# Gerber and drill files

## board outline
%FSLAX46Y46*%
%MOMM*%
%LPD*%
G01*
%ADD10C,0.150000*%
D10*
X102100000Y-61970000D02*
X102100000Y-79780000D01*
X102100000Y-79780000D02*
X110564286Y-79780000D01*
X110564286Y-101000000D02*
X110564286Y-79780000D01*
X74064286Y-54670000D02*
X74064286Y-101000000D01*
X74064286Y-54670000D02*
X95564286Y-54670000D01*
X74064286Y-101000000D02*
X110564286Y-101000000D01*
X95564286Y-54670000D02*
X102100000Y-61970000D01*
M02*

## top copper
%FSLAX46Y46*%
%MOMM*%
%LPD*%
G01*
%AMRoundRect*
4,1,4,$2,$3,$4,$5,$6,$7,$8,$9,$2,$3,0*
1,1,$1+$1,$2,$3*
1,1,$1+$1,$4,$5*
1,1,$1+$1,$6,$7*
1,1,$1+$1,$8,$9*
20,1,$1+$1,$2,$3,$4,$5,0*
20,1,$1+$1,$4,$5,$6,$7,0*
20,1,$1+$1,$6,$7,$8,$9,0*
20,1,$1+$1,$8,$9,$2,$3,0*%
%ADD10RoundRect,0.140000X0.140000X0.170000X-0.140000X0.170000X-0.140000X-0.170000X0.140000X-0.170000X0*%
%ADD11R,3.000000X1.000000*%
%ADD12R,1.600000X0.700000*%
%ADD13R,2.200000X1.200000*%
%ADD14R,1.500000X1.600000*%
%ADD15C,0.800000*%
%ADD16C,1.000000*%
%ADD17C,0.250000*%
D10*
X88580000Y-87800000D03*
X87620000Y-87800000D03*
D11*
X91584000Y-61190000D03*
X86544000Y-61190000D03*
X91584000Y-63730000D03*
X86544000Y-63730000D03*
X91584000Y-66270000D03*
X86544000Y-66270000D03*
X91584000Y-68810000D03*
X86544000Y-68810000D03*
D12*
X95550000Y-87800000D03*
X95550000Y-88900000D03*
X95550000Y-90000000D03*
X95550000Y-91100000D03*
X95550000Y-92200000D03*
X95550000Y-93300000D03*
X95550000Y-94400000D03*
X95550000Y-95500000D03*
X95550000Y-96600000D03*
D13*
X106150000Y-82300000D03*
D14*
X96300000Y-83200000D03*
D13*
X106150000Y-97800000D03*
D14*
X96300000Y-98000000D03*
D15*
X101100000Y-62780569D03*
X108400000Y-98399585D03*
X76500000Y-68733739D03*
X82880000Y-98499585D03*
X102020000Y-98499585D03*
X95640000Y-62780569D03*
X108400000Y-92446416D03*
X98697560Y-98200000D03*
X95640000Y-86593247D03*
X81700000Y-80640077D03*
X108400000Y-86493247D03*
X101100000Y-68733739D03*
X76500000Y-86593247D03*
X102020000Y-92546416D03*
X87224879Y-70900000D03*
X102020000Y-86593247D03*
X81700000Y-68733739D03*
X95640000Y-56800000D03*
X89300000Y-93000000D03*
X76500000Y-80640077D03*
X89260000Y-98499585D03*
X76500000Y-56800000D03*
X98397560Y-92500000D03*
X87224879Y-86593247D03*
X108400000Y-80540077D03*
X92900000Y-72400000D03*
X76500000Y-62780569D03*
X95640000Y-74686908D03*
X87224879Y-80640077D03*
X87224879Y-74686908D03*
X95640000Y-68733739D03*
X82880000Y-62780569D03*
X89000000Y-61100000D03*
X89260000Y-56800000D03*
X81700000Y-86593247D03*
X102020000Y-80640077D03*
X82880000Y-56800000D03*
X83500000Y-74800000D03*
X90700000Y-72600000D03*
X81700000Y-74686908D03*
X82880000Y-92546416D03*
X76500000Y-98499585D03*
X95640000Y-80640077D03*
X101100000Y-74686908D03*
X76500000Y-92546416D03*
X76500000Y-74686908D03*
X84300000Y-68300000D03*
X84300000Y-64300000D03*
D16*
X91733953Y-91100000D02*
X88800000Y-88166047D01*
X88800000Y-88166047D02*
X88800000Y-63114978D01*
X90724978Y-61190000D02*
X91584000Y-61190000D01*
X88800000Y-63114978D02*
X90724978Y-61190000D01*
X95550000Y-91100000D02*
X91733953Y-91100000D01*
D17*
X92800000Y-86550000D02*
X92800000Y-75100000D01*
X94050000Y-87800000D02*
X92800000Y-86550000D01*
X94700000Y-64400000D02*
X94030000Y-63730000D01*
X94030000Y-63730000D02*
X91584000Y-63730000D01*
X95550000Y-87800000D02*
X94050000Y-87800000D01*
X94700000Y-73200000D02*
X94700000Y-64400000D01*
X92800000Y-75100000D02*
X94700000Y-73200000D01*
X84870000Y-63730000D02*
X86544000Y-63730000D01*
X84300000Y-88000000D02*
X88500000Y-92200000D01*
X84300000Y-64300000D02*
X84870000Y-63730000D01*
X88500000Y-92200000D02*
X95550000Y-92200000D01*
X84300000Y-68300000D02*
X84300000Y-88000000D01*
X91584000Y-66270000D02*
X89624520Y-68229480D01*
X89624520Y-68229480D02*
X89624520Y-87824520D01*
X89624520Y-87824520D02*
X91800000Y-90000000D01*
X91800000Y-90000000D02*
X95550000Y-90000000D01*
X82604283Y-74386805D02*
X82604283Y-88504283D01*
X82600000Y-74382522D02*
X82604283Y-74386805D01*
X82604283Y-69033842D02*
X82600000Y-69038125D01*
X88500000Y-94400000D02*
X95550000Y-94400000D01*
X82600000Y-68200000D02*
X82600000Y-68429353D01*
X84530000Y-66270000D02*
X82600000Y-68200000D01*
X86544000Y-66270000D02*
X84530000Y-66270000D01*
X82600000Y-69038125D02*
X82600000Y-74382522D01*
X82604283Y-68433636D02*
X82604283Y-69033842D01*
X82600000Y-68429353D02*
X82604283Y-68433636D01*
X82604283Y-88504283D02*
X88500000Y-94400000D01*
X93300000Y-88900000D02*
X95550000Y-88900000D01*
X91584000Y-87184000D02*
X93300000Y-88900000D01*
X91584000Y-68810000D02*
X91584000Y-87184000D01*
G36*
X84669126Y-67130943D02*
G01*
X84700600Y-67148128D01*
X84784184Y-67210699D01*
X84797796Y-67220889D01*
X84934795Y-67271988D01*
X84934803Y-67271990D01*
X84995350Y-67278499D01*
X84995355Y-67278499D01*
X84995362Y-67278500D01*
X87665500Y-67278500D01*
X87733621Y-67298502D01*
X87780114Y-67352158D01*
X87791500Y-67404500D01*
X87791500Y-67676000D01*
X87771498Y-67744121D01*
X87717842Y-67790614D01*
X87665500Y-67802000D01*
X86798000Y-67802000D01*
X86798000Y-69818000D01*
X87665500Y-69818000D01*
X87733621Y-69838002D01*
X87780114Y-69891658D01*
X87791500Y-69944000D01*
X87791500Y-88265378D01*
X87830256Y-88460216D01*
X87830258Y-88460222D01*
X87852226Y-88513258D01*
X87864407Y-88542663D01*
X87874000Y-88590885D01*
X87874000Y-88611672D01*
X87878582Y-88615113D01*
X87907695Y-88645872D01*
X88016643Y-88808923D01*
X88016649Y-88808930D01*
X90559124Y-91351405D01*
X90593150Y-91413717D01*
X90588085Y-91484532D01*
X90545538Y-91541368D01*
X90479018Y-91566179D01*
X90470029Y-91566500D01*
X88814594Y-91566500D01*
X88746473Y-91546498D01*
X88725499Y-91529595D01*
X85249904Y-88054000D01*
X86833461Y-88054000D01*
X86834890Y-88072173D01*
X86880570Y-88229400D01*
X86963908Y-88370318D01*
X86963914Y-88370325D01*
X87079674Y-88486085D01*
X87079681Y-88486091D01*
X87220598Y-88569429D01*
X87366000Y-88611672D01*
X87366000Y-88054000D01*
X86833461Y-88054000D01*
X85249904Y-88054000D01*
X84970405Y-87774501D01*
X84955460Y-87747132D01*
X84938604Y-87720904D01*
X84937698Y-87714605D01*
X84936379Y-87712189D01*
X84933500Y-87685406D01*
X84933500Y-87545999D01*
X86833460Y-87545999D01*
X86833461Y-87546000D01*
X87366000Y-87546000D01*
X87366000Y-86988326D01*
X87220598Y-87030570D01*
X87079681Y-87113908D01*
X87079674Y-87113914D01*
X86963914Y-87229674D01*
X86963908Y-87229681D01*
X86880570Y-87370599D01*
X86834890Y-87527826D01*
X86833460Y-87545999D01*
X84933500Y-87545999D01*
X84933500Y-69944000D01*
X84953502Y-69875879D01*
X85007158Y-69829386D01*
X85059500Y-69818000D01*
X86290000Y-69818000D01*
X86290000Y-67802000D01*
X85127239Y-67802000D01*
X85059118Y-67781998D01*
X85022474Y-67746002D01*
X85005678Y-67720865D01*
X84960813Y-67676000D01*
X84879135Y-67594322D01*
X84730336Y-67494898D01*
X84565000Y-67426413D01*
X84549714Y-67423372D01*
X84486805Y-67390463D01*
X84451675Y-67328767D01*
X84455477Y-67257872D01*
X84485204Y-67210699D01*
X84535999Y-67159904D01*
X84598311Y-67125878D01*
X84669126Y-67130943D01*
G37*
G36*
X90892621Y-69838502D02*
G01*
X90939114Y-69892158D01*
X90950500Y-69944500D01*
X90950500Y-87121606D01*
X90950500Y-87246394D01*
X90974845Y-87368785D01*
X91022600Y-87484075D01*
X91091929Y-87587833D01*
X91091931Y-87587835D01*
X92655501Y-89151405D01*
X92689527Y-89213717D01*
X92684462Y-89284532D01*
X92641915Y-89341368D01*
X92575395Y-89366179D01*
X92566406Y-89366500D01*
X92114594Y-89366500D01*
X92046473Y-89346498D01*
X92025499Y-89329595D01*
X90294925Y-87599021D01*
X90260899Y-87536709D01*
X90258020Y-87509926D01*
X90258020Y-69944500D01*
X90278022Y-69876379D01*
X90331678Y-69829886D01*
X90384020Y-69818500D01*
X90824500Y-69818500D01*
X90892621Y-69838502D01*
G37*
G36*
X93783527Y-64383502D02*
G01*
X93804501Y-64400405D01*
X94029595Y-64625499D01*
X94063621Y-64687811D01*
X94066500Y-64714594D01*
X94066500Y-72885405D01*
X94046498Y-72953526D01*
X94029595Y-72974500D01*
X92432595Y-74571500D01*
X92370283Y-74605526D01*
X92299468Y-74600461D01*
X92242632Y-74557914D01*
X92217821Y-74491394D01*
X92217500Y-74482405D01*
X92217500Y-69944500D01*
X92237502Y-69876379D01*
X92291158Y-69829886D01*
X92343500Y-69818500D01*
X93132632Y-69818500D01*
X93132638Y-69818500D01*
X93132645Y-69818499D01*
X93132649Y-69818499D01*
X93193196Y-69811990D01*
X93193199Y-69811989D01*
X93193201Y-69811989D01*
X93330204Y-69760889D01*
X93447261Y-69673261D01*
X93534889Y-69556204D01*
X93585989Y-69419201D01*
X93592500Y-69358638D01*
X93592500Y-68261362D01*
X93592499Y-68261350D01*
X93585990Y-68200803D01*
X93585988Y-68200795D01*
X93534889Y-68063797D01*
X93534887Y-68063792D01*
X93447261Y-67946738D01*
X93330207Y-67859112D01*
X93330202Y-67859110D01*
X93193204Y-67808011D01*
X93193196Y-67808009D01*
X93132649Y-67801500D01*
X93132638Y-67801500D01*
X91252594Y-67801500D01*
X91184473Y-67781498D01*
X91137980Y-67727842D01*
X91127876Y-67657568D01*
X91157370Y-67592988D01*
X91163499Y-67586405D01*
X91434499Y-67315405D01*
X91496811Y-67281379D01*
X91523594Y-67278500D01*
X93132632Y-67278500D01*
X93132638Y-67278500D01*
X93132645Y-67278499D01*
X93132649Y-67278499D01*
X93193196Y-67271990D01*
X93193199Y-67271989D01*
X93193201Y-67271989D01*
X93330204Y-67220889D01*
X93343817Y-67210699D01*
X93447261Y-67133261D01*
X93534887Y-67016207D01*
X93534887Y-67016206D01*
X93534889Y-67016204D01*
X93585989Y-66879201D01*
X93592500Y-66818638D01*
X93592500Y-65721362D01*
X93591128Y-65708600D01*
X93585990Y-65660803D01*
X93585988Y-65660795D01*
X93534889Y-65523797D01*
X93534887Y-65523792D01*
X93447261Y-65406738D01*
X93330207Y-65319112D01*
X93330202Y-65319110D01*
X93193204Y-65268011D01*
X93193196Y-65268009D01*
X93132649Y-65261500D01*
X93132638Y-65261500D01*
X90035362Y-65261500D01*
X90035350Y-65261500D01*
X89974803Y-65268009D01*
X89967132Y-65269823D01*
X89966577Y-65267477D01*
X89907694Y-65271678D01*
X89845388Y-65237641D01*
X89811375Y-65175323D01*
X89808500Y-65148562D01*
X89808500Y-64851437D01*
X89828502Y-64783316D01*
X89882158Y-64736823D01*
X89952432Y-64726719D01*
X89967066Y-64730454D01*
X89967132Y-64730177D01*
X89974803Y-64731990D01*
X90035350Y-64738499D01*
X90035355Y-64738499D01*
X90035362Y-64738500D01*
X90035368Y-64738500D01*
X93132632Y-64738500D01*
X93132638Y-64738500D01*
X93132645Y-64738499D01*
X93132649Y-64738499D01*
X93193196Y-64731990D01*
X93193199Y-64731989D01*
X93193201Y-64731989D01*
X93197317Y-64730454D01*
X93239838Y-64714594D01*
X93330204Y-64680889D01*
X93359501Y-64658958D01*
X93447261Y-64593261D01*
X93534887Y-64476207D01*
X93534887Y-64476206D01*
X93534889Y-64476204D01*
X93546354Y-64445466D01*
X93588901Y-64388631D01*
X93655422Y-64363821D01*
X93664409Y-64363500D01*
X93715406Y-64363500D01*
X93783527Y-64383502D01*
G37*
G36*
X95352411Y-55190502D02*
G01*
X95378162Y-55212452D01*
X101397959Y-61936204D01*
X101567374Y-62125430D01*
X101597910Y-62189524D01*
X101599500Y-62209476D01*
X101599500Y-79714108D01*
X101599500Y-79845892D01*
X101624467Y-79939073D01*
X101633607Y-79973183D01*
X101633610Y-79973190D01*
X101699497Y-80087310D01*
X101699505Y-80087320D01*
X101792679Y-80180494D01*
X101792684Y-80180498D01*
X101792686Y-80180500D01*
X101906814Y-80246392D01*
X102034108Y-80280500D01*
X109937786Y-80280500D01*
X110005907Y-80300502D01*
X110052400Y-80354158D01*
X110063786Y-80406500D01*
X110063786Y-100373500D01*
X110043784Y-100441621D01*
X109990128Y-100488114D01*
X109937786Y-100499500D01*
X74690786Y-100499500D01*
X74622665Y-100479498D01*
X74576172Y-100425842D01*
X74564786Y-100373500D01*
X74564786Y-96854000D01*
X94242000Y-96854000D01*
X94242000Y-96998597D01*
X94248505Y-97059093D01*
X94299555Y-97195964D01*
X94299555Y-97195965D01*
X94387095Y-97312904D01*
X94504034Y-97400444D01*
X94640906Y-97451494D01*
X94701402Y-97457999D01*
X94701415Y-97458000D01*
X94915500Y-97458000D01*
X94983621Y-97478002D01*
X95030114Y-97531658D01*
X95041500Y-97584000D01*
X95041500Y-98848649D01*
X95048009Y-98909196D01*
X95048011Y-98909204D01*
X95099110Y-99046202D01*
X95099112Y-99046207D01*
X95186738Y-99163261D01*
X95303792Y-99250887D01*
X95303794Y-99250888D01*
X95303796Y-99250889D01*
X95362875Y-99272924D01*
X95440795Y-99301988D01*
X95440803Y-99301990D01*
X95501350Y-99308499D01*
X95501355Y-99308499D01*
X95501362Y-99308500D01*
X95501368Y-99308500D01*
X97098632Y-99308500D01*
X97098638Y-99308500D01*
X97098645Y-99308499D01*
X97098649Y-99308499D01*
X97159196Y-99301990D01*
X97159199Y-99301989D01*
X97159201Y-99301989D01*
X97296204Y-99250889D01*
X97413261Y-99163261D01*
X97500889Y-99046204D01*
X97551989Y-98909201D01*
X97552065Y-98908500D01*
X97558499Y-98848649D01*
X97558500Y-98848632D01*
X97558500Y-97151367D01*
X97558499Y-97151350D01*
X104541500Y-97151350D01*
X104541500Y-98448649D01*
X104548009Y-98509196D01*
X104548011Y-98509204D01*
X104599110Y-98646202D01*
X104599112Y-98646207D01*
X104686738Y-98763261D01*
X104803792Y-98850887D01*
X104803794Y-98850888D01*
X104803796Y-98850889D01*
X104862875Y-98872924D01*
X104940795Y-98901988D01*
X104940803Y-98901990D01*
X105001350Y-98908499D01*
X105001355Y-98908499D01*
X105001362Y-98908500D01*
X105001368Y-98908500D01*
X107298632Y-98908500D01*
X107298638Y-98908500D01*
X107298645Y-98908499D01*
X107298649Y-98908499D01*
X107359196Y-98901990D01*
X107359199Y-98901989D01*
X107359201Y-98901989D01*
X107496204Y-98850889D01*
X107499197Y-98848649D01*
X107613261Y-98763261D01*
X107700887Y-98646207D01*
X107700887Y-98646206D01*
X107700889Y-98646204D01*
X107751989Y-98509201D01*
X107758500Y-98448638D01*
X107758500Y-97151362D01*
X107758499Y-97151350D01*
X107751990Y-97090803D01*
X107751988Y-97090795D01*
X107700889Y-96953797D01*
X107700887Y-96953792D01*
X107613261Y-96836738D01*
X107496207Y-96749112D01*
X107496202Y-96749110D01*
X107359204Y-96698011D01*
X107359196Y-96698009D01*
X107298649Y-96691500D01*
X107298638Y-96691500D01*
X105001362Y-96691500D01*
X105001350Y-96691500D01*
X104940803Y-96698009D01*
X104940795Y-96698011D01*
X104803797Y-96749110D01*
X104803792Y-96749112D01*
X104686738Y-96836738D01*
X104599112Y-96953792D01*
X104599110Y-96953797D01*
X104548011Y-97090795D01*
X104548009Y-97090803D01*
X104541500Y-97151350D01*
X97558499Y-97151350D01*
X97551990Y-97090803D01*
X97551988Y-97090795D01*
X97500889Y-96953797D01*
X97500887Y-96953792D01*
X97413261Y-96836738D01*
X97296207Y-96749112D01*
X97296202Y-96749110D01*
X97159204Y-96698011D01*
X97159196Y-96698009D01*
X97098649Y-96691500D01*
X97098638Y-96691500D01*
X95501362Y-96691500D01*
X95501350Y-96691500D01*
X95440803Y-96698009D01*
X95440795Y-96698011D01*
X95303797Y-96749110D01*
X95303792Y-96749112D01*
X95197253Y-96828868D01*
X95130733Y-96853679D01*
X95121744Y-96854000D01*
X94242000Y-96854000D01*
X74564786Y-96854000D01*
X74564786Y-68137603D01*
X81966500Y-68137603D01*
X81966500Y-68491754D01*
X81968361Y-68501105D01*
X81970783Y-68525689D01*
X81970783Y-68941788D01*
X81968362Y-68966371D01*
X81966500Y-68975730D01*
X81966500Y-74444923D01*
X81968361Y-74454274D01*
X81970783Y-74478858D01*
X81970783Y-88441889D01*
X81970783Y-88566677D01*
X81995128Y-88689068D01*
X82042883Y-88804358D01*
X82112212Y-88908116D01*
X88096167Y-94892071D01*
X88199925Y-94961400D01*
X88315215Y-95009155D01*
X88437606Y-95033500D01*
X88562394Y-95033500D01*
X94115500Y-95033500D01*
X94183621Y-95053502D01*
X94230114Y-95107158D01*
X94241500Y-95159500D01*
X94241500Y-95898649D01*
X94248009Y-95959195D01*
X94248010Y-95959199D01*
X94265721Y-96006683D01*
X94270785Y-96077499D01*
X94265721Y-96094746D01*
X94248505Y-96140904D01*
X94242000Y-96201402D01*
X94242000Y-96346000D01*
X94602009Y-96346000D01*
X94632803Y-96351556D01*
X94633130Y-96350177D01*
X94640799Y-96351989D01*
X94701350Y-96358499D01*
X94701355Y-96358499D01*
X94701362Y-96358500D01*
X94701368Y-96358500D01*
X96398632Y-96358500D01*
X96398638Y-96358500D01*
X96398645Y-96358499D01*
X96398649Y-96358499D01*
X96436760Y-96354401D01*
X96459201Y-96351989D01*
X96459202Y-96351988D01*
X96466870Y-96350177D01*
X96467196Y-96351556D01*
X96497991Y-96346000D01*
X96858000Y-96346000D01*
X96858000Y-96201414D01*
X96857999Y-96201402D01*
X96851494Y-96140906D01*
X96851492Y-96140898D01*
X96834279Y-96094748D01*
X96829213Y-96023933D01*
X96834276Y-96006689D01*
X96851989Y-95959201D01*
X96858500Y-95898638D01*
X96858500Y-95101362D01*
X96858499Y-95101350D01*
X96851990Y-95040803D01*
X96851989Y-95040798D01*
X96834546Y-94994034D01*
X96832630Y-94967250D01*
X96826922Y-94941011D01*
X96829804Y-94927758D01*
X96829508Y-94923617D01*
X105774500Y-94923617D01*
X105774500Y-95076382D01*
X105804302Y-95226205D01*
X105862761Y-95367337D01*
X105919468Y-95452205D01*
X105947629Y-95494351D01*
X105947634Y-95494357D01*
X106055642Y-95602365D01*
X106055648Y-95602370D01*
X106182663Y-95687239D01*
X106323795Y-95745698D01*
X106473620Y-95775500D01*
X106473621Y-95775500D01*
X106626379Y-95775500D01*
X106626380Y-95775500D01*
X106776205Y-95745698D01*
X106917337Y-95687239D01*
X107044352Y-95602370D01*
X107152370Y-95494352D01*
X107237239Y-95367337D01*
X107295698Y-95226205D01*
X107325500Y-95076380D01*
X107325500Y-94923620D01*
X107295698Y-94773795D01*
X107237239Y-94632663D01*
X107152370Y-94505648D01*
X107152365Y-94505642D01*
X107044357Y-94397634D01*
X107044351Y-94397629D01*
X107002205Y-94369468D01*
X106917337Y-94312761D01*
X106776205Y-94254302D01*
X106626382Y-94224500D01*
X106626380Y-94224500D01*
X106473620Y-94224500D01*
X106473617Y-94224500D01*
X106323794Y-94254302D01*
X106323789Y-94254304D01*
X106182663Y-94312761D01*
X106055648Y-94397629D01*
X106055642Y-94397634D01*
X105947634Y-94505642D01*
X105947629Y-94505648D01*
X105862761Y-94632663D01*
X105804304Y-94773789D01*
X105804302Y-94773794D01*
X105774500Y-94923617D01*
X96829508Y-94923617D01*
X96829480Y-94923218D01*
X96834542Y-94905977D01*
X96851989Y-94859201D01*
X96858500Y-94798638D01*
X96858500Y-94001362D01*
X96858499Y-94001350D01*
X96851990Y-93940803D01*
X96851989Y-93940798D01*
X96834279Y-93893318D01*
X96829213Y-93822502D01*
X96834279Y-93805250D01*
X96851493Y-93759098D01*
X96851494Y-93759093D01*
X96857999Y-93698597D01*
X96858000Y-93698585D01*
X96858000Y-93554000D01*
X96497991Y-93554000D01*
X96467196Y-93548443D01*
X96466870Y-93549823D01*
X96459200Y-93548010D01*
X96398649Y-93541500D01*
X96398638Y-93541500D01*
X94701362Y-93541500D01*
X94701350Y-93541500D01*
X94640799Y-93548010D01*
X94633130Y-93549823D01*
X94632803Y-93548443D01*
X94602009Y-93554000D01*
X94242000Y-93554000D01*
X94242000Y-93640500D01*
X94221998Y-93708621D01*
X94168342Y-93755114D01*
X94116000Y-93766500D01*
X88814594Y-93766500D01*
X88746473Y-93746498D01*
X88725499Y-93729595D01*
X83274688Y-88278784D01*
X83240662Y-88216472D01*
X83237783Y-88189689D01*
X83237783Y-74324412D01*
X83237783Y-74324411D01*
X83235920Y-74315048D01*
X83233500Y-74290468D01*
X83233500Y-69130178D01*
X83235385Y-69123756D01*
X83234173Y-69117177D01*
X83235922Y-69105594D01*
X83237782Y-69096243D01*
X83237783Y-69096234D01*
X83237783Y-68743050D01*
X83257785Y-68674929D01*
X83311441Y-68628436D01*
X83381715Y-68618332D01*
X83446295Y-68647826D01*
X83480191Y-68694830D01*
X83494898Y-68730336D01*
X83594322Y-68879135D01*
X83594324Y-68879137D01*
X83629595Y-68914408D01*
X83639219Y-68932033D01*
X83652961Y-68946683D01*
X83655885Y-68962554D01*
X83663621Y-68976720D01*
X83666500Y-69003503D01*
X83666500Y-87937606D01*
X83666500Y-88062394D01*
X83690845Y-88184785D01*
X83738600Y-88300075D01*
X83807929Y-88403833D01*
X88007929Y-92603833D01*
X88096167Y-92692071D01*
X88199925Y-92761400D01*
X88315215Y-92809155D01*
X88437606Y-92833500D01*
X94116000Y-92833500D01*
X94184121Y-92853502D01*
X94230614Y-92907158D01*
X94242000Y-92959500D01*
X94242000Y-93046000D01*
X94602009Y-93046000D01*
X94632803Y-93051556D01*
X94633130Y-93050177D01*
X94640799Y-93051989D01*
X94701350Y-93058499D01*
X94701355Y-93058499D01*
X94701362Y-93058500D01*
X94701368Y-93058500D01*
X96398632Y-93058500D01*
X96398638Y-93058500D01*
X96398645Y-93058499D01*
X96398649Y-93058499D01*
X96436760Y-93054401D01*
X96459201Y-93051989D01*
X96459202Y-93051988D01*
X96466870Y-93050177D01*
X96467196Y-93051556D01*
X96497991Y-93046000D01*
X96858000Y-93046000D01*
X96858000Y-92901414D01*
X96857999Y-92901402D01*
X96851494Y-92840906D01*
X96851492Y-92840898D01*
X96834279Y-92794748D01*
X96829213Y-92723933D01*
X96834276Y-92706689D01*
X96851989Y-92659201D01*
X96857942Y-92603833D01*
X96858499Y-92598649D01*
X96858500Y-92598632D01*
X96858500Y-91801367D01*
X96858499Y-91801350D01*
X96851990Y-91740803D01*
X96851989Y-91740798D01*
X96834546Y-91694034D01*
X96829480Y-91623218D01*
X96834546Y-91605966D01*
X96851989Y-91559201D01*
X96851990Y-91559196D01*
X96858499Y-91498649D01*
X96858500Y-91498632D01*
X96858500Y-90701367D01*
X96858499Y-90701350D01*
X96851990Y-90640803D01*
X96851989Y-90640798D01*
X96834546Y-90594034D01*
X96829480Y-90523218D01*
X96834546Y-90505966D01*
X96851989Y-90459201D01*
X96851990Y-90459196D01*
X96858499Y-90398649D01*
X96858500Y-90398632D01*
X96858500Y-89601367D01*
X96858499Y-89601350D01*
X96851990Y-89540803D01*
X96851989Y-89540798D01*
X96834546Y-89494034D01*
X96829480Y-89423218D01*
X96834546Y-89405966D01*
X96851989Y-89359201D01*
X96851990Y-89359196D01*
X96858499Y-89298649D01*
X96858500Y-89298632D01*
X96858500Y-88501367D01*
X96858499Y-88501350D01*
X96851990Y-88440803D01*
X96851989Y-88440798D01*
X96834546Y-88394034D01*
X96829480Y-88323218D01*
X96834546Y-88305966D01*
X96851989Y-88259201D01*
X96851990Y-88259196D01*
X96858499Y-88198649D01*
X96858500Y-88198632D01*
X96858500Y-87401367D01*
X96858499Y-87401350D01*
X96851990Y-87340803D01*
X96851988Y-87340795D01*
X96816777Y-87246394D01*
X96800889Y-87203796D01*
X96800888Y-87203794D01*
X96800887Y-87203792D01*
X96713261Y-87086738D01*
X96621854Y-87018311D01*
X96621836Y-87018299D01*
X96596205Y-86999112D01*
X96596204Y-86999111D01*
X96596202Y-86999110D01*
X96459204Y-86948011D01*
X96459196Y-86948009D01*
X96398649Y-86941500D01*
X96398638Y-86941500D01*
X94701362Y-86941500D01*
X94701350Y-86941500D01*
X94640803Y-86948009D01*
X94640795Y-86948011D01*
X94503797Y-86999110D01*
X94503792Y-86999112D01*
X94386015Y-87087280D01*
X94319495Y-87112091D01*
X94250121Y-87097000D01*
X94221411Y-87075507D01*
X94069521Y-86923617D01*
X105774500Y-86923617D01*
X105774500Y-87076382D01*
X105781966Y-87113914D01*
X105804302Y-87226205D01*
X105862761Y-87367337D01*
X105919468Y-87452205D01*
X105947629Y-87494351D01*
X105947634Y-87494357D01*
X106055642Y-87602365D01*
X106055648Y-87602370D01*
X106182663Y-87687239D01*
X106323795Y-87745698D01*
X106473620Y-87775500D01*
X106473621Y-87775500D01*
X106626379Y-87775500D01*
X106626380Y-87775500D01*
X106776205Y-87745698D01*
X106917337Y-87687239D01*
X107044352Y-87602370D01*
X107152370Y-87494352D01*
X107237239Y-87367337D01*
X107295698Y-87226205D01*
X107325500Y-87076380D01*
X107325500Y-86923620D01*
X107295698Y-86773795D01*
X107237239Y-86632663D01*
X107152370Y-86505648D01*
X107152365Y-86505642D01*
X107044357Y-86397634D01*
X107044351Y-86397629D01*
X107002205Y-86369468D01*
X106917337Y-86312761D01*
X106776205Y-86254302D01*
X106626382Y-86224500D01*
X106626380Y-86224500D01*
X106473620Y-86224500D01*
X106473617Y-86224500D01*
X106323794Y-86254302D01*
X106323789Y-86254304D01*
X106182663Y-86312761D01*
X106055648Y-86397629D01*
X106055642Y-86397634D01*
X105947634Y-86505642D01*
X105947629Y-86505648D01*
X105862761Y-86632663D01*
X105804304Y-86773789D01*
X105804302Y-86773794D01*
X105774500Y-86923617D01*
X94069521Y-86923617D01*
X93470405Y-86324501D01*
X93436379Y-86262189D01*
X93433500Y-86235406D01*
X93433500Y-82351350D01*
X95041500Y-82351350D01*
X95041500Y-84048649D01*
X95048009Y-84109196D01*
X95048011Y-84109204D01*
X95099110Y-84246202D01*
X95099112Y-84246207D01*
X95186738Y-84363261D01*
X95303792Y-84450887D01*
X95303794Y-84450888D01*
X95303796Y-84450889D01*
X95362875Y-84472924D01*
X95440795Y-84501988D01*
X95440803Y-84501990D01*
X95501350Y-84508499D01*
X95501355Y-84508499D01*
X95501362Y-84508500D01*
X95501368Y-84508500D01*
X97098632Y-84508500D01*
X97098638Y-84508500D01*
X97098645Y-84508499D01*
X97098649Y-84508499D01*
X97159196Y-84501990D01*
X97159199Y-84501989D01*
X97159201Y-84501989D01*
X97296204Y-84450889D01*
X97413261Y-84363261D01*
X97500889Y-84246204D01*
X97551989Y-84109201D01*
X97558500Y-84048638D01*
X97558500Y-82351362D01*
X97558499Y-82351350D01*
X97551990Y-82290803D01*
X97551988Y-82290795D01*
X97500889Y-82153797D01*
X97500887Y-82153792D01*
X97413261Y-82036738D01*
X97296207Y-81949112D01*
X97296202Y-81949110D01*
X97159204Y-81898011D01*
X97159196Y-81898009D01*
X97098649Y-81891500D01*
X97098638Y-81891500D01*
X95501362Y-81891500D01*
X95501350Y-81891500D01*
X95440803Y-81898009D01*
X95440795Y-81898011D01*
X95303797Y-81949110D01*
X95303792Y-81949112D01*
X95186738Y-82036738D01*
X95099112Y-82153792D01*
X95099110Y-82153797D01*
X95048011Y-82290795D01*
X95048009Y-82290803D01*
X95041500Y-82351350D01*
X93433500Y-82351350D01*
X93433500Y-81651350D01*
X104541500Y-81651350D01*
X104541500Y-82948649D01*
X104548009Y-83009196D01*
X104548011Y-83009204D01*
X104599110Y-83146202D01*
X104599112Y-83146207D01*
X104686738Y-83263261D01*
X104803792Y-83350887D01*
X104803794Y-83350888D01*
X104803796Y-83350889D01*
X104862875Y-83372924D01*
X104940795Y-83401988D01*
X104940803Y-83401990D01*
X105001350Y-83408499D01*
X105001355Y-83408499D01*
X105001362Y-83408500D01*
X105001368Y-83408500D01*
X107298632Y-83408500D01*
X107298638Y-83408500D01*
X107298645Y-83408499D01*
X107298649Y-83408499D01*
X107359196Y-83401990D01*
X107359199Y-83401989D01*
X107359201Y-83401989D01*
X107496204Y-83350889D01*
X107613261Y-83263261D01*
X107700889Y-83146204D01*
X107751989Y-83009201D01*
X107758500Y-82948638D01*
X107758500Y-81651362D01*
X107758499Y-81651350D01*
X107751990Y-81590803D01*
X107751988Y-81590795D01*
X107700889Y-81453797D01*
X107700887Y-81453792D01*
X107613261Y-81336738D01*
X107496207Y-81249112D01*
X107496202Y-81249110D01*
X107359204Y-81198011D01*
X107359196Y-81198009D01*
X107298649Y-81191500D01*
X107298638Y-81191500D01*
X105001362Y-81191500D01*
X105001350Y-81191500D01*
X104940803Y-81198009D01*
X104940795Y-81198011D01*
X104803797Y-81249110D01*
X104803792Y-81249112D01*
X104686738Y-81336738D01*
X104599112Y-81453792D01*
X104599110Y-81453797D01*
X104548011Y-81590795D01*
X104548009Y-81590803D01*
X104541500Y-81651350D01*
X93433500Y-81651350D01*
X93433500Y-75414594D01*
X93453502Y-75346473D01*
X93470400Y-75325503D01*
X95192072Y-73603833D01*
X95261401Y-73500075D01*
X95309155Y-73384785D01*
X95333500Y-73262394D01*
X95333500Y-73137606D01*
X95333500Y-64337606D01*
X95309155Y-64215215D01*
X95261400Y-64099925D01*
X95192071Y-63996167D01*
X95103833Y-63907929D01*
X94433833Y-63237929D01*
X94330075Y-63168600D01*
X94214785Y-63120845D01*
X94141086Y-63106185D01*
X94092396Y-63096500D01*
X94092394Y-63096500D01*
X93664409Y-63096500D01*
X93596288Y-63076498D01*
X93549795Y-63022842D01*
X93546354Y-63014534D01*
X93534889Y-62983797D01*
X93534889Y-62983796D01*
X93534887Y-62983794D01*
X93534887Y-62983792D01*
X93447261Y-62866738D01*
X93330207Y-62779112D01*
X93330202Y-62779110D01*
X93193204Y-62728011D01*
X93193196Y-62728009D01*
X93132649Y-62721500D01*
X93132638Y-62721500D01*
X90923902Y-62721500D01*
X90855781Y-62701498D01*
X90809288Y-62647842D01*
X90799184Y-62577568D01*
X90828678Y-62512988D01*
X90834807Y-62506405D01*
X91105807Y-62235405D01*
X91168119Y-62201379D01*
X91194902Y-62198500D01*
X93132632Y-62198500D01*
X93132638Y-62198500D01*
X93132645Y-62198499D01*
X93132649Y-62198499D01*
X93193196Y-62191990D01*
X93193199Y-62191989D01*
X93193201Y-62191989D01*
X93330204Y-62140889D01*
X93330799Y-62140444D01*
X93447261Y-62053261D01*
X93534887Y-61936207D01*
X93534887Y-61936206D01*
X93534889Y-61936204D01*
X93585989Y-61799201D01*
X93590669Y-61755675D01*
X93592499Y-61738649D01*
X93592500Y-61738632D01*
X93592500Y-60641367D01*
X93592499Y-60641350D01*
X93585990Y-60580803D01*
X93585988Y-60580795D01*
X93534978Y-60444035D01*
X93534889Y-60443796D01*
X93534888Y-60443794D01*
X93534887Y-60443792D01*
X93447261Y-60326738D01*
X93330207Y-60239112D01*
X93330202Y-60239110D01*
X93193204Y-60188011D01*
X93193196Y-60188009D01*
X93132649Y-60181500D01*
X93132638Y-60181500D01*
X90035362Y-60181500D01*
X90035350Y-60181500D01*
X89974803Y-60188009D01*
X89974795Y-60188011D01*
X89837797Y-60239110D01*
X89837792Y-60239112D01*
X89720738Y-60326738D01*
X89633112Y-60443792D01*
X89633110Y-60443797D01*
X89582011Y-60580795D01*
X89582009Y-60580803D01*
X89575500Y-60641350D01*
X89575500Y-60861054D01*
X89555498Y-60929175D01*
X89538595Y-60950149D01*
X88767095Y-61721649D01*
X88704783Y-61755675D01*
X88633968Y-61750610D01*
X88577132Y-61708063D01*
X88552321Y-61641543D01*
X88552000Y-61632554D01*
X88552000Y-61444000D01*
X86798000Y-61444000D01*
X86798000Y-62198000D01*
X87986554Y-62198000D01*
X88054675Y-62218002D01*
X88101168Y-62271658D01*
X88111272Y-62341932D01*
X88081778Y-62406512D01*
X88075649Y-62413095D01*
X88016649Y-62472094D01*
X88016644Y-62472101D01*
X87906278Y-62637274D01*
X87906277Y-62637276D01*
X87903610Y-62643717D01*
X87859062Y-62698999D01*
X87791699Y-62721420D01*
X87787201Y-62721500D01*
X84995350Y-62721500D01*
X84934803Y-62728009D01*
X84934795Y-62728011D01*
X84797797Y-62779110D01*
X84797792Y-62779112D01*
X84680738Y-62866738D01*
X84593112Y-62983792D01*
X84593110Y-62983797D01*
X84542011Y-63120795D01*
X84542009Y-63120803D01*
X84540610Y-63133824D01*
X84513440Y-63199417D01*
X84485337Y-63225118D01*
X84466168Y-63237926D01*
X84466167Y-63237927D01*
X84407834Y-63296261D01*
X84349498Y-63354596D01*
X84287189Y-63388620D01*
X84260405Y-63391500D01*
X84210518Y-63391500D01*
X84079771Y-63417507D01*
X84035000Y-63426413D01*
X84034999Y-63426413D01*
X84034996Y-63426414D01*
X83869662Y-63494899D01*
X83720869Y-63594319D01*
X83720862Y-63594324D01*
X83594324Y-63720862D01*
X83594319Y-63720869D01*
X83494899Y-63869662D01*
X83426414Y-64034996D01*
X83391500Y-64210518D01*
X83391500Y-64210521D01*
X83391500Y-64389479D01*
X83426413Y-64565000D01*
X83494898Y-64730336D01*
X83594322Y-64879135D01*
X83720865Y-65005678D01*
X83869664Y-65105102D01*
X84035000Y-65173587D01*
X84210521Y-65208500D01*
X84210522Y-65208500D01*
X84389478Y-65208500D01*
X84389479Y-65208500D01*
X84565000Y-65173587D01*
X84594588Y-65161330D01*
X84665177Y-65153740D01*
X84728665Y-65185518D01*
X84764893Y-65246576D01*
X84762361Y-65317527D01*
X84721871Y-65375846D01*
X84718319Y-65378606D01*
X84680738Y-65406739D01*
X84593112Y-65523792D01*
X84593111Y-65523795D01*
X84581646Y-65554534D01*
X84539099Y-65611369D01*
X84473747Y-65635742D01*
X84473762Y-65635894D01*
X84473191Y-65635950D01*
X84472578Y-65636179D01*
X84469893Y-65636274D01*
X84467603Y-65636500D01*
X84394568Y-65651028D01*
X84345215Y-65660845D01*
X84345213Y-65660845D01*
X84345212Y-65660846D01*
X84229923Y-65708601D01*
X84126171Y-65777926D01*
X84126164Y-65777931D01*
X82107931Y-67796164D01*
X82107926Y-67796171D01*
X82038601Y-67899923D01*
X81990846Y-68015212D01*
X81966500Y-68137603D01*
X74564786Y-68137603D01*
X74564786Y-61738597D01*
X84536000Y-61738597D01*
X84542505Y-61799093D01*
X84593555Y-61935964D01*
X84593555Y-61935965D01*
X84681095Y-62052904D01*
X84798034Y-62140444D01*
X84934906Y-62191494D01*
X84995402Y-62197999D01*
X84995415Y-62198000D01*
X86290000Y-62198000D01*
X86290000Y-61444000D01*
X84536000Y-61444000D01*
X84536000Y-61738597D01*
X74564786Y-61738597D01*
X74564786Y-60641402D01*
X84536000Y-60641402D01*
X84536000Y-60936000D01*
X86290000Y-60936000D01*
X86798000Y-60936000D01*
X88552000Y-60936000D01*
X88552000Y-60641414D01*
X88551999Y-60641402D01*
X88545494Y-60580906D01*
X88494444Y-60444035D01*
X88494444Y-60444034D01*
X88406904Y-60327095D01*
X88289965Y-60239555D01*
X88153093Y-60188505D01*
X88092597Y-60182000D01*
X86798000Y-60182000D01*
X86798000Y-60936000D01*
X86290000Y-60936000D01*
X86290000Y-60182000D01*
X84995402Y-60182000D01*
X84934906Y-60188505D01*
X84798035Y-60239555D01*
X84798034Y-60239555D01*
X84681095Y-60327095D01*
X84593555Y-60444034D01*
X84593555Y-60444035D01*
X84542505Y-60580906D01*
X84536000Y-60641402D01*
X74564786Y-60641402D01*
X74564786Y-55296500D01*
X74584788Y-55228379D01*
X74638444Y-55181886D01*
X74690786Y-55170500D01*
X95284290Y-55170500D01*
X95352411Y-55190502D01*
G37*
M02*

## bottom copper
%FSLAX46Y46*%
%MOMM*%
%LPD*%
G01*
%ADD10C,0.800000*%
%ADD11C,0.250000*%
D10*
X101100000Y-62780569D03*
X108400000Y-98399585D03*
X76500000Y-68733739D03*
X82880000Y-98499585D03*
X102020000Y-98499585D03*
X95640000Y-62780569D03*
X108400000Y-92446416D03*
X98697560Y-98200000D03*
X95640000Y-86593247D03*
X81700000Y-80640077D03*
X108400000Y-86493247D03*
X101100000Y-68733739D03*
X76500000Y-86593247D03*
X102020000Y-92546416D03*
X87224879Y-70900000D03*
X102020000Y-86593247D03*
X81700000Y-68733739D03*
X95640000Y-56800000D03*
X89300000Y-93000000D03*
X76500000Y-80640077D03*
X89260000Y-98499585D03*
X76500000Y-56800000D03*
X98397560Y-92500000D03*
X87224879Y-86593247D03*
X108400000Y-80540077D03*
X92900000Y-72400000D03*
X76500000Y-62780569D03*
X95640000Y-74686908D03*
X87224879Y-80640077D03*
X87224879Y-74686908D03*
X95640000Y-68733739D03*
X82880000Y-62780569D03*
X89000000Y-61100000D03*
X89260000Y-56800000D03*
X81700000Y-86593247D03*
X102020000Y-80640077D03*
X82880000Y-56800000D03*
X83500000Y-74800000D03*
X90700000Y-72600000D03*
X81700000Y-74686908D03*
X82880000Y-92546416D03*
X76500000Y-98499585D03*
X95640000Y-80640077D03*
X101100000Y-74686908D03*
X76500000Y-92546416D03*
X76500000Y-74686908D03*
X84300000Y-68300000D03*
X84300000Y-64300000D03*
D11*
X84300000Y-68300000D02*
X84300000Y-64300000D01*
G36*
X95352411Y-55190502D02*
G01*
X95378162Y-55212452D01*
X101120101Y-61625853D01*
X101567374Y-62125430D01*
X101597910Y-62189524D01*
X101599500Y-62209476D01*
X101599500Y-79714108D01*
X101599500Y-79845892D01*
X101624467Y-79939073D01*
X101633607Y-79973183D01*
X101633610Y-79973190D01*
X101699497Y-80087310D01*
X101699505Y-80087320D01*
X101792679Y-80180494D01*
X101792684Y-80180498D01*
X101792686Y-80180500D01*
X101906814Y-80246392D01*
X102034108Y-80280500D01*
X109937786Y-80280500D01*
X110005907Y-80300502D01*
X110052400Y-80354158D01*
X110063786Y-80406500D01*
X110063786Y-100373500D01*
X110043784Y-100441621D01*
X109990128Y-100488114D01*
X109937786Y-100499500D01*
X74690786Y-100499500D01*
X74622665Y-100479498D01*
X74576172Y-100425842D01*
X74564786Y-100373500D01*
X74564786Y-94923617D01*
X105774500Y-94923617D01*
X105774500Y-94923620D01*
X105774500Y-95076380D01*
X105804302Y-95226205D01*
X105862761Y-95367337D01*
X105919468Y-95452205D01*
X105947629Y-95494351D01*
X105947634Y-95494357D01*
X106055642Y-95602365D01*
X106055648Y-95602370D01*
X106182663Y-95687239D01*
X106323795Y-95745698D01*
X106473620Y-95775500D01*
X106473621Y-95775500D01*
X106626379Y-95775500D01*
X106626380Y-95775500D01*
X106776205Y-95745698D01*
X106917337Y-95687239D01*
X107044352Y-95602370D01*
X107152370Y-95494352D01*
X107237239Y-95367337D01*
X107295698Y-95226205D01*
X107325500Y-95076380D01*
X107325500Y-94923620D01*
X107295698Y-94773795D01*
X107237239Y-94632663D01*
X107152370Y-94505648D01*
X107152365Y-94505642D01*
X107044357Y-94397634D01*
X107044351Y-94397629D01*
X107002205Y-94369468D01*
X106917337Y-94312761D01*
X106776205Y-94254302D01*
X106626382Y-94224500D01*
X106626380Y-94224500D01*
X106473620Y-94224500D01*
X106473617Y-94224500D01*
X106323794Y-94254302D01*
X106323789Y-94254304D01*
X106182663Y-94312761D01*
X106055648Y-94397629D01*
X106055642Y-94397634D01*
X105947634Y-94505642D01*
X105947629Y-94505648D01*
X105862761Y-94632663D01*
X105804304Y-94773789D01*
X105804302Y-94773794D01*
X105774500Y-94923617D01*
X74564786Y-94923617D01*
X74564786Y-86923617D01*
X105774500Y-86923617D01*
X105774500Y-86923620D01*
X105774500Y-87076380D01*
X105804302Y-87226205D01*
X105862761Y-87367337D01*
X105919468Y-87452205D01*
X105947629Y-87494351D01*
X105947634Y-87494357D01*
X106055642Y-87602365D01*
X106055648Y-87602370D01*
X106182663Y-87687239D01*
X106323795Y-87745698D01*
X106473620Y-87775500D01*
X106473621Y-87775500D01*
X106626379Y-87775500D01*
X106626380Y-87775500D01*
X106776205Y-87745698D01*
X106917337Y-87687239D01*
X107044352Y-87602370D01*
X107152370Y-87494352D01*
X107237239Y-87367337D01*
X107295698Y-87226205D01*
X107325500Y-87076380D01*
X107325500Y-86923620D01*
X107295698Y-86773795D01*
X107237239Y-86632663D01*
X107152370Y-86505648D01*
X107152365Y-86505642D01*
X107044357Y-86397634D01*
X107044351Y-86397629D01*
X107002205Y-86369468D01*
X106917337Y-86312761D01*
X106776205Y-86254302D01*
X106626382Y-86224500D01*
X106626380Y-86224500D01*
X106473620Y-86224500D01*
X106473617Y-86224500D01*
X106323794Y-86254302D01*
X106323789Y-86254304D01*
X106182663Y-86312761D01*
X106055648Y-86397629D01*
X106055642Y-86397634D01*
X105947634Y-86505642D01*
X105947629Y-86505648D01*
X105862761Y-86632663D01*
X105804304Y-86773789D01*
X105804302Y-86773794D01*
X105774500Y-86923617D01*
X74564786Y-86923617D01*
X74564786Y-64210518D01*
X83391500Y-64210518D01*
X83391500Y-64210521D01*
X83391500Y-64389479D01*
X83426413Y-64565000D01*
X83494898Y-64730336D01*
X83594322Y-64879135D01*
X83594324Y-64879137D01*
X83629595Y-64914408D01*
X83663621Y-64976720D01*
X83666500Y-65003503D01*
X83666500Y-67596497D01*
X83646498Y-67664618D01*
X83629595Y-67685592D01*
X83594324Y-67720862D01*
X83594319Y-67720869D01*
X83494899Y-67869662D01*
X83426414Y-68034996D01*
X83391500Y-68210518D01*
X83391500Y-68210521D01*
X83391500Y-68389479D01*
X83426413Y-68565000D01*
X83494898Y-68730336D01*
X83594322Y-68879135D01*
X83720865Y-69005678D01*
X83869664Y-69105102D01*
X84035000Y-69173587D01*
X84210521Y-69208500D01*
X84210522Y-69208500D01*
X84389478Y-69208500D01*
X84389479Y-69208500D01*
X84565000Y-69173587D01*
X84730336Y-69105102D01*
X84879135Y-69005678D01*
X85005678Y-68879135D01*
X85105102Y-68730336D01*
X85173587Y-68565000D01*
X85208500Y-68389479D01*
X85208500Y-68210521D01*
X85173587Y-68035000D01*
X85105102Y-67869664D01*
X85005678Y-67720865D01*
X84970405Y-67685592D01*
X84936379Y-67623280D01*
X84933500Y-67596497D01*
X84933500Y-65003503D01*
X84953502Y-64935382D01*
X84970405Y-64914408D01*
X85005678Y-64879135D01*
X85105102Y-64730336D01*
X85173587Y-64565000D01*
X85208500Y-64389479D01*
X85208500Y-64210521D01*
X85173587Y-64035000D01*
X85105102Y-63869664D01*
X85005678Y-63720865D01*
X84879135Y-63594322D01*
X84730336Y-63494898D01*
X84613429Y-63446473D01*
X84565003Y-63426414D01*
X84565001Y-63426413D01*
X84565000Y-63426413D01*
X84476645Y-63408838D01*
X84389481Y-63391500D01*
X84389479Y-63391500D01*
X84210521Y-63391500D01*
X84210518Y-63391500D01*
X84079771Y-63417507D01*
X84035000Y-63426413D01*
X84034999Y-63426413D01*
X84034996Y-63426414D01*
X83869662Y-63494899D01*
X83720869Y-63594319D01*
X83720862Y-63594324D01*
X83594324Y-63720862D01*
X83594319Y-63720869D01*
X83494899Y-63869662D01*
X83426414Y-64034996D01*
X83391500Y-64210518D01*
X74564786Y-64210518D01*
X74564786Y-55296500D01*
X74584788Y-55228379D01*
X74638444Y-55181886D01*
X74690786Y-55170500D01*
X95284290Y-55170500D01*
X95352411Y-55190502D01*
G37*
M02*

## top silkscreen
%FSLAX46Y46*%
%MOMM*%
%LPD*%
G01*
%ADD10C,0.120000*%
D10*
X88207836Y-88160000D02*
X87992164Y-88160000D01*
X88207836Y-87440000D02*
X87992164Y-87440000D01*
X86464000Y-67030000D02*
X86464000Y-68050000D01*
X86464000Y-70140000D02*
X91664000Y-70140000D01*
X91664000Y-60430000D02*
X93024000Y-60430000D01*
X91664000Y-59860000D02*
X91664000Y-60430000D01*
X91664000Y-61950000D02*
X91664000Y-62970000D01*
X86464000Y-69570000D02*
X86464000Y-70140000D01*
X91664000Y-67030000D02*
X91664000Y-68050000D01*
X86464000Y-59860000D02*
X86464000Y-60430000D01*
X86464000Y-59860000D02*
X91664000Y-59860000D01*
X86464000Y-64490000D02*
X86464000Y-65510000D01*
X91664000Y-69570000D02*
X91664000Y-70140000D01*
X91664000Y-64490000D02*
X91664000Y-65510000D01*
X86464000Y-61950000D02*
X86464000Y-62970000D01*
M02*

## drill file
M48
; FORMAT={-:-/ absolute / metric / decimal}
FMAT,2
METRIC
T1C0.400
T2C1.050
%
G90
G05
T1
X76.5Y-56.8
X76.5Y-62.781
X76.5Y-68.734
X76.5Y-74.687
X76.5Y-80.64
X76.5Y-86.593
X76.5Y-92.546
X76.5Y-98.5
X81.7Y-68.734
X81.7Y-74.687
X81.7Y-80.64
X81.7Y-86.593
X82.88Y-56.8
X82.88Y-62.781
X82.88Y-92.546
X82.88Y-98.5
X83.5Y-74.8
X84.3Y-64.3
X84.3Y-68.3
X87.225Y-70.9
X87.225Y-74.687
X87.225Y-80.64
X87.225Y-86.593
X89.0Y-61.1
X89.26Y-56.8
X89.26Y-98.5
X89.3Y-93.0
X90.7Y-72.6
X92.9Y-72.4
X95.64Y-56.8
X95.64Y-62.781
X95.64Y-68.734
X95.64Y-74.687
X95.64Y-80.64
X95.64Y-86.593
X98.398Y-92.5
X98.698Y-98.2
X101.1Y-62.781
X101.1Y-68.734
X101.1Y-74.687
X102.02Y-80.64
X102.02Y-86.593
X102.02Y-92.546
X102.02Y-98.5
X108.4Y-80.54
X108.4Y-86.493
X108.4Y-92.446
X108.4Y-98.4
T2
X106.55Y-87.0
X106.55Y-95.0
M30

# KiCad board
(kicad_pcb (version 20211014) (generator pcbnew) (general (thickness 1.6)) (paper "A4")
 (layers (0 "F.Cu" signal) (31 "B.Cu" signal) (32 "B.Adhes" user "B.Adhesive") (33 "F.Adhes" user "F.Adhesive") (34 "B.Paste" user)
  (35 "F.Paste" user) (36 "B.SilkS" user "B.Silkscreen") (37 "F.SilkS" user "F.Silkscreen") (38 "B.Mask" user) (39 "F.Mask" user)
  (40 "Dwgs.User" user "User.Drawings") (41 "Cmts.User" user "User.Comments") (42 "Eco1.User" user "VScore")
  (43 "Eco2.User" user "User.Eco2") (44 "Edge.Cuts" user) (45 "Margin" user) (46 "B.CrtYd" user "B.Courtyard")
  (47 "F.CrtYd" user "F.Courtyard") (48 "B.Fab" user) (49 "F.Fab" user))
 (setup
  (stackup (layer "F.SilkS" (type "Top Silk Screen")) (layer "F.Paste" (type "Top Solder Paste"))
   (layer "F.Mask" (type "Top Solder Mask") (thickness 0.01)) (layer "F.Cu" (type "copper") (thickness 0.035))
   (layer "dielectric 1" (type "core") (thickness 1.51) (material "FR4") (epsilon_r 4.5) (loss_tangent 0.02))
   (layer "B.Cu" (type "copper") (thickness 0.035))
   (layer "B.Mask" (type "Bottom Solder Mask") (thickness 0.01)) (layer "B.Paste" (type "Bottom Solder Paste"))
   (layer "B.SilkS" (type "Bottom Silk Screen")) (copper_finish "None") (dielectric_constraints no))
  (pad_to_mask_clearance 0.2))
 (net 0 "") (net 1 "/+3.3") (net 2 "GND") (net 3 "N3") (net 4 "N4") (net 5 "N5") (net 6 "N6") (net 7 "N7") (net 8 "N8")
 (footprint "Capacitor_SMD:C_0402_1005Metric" (layer "F.Cu") (at 88.1 87.8 180)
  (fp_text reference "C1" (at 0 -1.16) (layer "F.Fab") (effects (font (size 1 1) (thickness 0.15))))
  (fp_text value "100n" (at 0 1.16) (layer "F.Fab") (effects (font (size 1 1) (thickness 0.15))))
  (fp_line (start -0.107836 -0.36) (end 0.107836 -0.36) (layer "F.SilkS") (width 0.12))
  (fp_line (start -0.107836 0.36) (end 0.107836 0.36) (layer "F.SilkS") (width 0.12))
  (pad "1" smd roundrect (at -0.48 0 180) (size 0.56 0.62) (layers "F.Cu" "F.Paste" "F.Mask") (roundrect_rratio 0.25) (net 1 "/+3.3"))
  (pad "2" smd roundrect (at 0.48 0 180) (size 0.56 0.62) (layers "F.Cu" "F.Paste" "F.Mask") (roundrect_rratio 0.25) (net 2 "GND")))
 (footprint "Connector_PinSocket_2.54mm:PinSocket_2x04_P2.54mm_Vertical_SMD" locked (layer "F.Cu") (at 89.064 65)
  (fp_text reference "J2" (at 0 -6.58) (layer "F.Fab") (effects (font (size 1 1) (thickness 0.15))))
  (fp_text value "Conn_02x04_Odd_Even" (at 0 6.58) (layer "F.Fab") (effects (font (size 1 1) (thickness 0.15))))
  (fp_line (start -2.6 2.03) (end -2.6 3.05) (layer "F.SilkS") (width 0.12))
  (fp_line (start -2.6 5.14) (end 2.6 5.14) (layer "F.SilkS") (width 0.12))
  (fp_line (start 2.6 -4.57) (end 3.96 -4.57) (layer "F.SilkS") (width 0.12))
  (fp_line (start 2.6 -5.14) (end 2.6 -4.57) (layer "F.SilkS") (width 0.12))
  (fp_line (start 2.6 -3.05) (end 2.6 -2.03) (layer "F.SilkS") (width 0.12))
  (fp_line (start -2.6 4.57) (end -2.6 5.14) (layer "F.SilkS") (width 0.12))
  (fp_line (start 2.6 2.03) (end 2.6 3.05) (layer "F.SilkS") (width 0.12))
  (fp_line (start -2.6 -5.14) (end -2.6 -4.57) (layer "F.SilkS") (width 0.12))
  (fp_line (start -2.6 -5.14) (end 2.6 -5.14) (layer "F.SilkS") (width 0.12))
  (fp_line (start -2.6 -0.51) (end -2.6 0.51) (layer "F.SilkS") (width 0.12))
  (fp_line (start 2.6 4.57) (end 2.6 5.14) (layer "F.SilkS") (width 0.12))
  (fp_line (start 2.6 -0.51) (end 2.6 0.51) (layer "F.SilkS") (width 0.12))
  (fp_line (start -2.6 -3.05) (end -2.6 -2.03) (layer "F.SilkS") (width 0.12))
  (pad "1" smd rect locked (at 2.52 -3.81) (size 3 1) (layers "F.Cu" "F.Paste" "F.Mask") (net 1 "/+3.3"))
  (pad "2" smd rect locked (at -2.52 -3.81) (size 3 1) (layers "F.Cu" "F.Paste" "F.Mask") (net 2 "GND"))
  (pad "3" smd rect locked (at 2.52 -1.27) (size 3 1) (layers "F.Cu" "F.Paste" "F.Mask") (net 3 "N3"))
  (pad "4" smd rect locked (at -2.52 -1.27) (size 3 1) (layers "F.Cu" "F.Paste" "F.Mask") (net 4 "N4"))
  (pad "5" smd rect locked (at 2.52 1.27) (size 3 1) (layers "F.Cu" "F.Paste" "F.Mask") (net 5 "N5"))
  (pad "6" smd rect locked (at -2.52 1.27) (size 3 1) (layers "F.Cu" "F.Paste" "F.Mask") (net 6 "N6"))
  (pad "7" smd rect locked (at 2.52 3.81) (size 3 1) (layers "F.Cu" "F.Paste" "F.Mask") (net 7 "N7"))
  (pad "8" smd rect locked (at -2.52 3.81) (size 3 1) (layers "F.Cu" "F.Paste" "F.Mask") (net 2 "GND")))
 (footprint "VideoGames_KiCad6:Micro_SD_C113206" (layer "F.Cu") (at 95.8 87.8 90)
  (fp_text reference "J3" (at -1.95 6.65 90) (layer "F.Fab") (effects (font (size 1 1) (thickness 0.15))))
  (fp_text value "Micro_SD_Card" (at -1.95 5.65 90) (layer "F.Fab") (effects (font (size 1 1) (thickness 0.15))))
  (pad "" np_thru_hole circle (at 0.8 10.75 90) (size 1.05 1.05) (drill 1.05) (layers *.Cu *.Mask))
  (pad "" np_thru_hole circle (at -7.2 10.75 90) (size 1.05 1.05) (drill 1.05) (layers *.Cu *.Mask))
  (pad "1" smd rect (at 0 -0.25 90) (size 0.7 1.6) (layers "F.Cu" "F.Paste" "F.Mask") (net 3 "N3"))
  (pad "2" smd rect (at -1.1 -0.25 90) (size 0.7 1.6) (layers "F.Cu" "F.Paste" "F.Mask") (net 7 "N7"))
  (pad "3" smd rect (at -2.2 -0.25 90) (size 0.7 1.6) (layers "F.Cu" "F.Paste" "F.Mask") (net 5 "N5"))
  (pad "4" smd rect (at -3.3 -0.25 90) (size 0.7 1.6) (layers "F.Cu" "F.Paste" "F.Mask") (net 1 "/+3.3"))
  (pad "5" smd rect (at -4.4 -0.25 90) (size 0.7 1.6) (layers "F.Cu" "F.Paste" "F.Mask") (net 4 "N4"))
  (pad "6" smd rect (at -5.5 -0.25 90) (size 0.7 1.6) (layers "F.Cu" "F.Paste" "F.Mask") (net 2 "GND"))
  (pad "7" smd rect (at -6.6 -0.25 90) (size 0.7 1.6) (layers "F.Cu" "F.Paste" "F.Mask") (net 6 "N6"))
  (pad "8" smd rect (at -7.7 -0.25 90) (size 0.7 1.6) (layers "F.Cu" "F.Paste" "F.Mask") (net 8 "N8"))
  (pad "9" smd rect (at -8.8 -0.25 90) (size 0.7 1.6) (layers "F.Cu" "F.Paste" "F.Mask") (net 2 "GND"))
  (pad "SH" smd rect (at 5.5 10.35 90) (size 1.2 2.2) (layers "F.Cu" "F.Paste" "F.Mask"))
  (pad "SH" smd rect (at 4.6 0.5 90) (size 1.6 1.5) (layers "F.Cu" "F.Paste" "F.Mask"))
  (pad "SH" smd rect (at -10 10.35 90) (size 1.2 2.2) (layers "F.Cu" "F.Paste" "F.Mask"))
  (pad "SH" smd rect (at -10.2 0.5 90) (size 1.6 1.5) (layers "F.Cu" "F.Paste" "F.Mask")))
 (gr_line (start 102.1 61.97) (end 102.1 79.78) (layer "Edge.Cuts") (width 0.15))
 (gr_line (start 102.1 79.78) (end 110.564286 79.78) (layer "Edge.Cuts") (width 0.15))
 (gr_line (start 110.564286 101) (end 110.564286 79.78) (layer "Edge.Cuts") (width 0.15))
 (gr_line (start 74.064286 54.67) (end 74.064286 101) (layer "Edge.Cuts") (width 0.15))
 (gr_line (start 74.064286 54.67) (end 95.564286 54.67) (layer "Edge.Cuts") (width 0.15))
 (gr_line (start 74.064286 101) (end 110.564286 101) (layer "Edge.Cuts") (width 0.15))
 (gr_line (start 95.564286 54.67) (end 102.1 61.97) (layer "Edge.Cuts") (width 0.15))
 (segment (start 91.733953 91.1) (end 88.8 88.166047) (width 1) (layer "F.Cu") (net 1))
 (segment (start 88.8 88.166047) (end 88.8 63.114978) (width 1) (layer "F.Cu") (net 1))
 (segment (start 90.724978 61.19) (end 91.584 61.19) (width 1) (layer "F.Cu") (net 1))
 (segment (start 88.8 63.114978) (end 90.724978 61.19) (width 1) (layer "F.Cu") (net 1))
 (segment (start 95.55 91.1) (end 91.733953 91.1) (width 1) (layer "F.Cu") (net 1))
 (via (at 101.1 62.780569) (size 0.8) (drill 0.4) (layers "F.Cu" "B.Cu") (free) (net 2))
 (via (at 108.4 98.399585) (size 0.8) (drill 0.4) (layers "F.Cu" "B.Cu") (free) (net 2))
 (via (at 76.5 68.733739) (size 0.8) (drill 0.4) (layers "F.Cu" "B.Cu") (free) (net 2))
 (via (at 82.88 98.499585) (size 0.8) (drill 0.4) (layers "F.Cu" "B.Cu") (free) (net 2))
 (via (at 102.02 98.499585) (size 0.8) (drill 0.4) (layers "F.Cu" "B.Cu") (free) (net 2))
 (via (at 95.64 62.780569) (size 0.8) (drill 0.4) (layers "F.Cu" "B.Cu") (free) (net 2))
 (via (at 108.4 92.446416) (size 0.8) (drill 0.4) (layers "F.Cu" "B.Cu") (free) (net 2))
 (via (at 98.69756 98.2) (size 0.8) (drill 0.4) (layers "F.Cu" "B.Cu") (free) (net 2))
 (via (at 95.64 86.593247) (size 0.8) (drill 0.4) (layers "F.Cu" "B.Cu") (free) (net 2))
 (via (at 81.7 80.640077) (size 0.8) (drill 0.4) (layers "F.Cu" "B.Cu") (free) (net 2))
 (via (at 108.4 86.493247) (size 0.8) (drill 0.4) (layers "F.Cu" "B.Cu") (free) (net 2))
 (via (at 101.1 68.733739) (size 0.8) (drill 0.4) (layers "F.Cu" "B.Cu") (free) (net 2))
 (via (at 76.5 86.593247) (size 0.8) (drill 0.4) (layers "F.Cu" "B.Cu") (free) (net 2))
 (via (at 102.02 92.546416) (size 0.8) (drill 0.4) (layers "F.Cu" "B.Cu") (free) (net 2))
 (via (at 87.224879 70.9) (size 0.8) (drill 0.4) (layers "F.Cu" "B.Cu") (free) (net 2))
 (via (at 102.02 86.593247) (size 0.8) (drill 0.4) (layers "F.Cu" "B.Cu") (free) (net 2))
 (via (at 81.7 68.733739) (size 0.8) (drill 0.4) (layers "F.Cu" "B.Cu") (free) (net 2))
 (via (at 95.64 56.8) (size 0.8) (drill 0.4) (layers "F.Cu" "B.Cu") (free) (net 2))
 (via (at 89.3 93) (size 0.8) (drill 0.4) (layers "F.Cu" "B.Cu") (free) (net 2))
 (via (at 76.5 80.640077) (size 0.8) (drill 0.4) (layers "F.Cu" "B.Cu") (free) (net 2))
 (via (at 89.26 98.499585) (size 0.8) (drill 0.4) (layers "F.Cu" "B.Cu") (free) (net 2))
 (via (at 76.5 56.8) (size 0.8) (drill 0.4) (layers "F.Cu" "B.Cu") (free) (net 2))
 (via (at 98.39756 92.5) (size 0.8) (drill 0.4) (layers "F.Cu" "B.Cu") (free) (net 2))
 (via (at 87.224879 86.593247) (size 0.8) (drill 0.4) (layers "F.Cu" "B.Cu") (free) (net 2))
 (via (at 108.4 80.540077) (size 0.8) (drill 0.4) (layers "F.Cu" "B.Cu") (free) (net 2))
 (via (at 92.9 72.4) (size 0.8) (drill 0.4) (layers "F.Cu" "B.Cu") (free) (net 2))
 (via (at 76.5 62.780569) (size 0.8) (drill 0.4) (layers "F.Cu" "B.Cu") (free) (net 2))
 (via (at 95.64 74.686908) (size 0.8) (drill 0.4) (layers "F.Cu" "B.Cu") (free) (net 2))
 (via (at 87.224879 80.640077) (size 0.8) (drill 0.4) (layers "F.Cu" "B.Cu") (free) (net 2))
 (via (at 87.224879 74.686908) (size 0.8) (drill 0.4) (layers "F.Cu" "B.Cu") (free) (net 2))
 (via (at 95.64 68.733739) (size 0.8) (drill 0.4) (layers "F.Cu" "B.Cu") (free) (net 2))
 (via (at 82.88 62.780569) (size 0.8) (drill 0.4) (layers "F.Cu" "B.Cu") (free) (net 2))
 (via (at 89 61.1) (size 0.8) (drill 0.4) (layers "F.Cu" "B.Cu") (free) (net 2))
 (via (at 89.26 56.8) (size 0.8) (drill 0.4) (layers "F.Cu" "B.Cu") (free) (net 2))
 (via (at 81.7 86.593247) (size 0.8) (drill 0.4) (layers "F.Cu" "B.Cu") (free) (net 2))
 (via (at 102.02 80.640077) (size 0.8) (drill 0.4) (layers "F.Cu" "B.Cu") (free) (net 2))
 (via (at 82.88 56.8) (size 0.8) (drill 0.4) (layers "F.Cu" "B.Cu") (free) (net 2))
 (via (at 83.5 74.8) (size 0.8) (drill 0.4) (layers "F.Cu" "B.Cu") (free) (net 2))
 (via (at 90.7 72.6) (size 0.8) (drill 0.4) (layers "F.Cu" "B.Cu") (free) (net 2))
 (via (at 81.7 74.686908) (size 0.8) (drill 0.4) (layers "F.Cu" "B.Cu") (free) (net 2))
 (via (at 82.88 92.546416) (size 0.8) (drill 0.4) (layers "F.Cu" "B.Cu") (free) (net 2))
 (via (at 76.5 98.499585) (size 0.8) (drill 0.4) (layers "F.Cu" "B.Cu") (free) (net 2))
 (via (at 95.64 80.640077) (size 0.8) (drill 0.4) (layers "F.Cu" "B.Cu") (free) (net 2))
 (via (at 101.1 74.686908) (size 0.8) (drill 0.4) (layers "F.Cu" "B.Cu") (free) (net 2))
 (via (at 76.5 92.546416) (size 0.8) (drill 0.4) (layers "F.Cu" "B.Cu") (free) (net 2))
 (via (at 76.5 74.686908) (size 0.8) (drill 0.4) (layers "F.Cu" "B.Cu") (free) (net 2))
 (segment (start 92.8 86.55) (end 92.8 75.1) (width 0.25) (layer "F.Cu") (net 3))
 (segment (start 94.05 87.8) (end 92.8 86.55) (width 0.25) (layer "F.Cu") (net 3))
 (segment (start 94.7 64.4) (end 94.03 63.73) (width 0.25) (layer "F.Cu") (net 3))
 (segment (start 94.03 63.73) (end 91.584 63.73) (width 0.25) (layer "F.Cu") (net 3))
 (segment (start 95.55 87.8) (end 94.05 87.8) (width 0.25) (layer "F.Cu") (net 3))
 (segment (start 94.7 73.2) (end 94.7 64.4) (width 0.25) (layer "F.Cu") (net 3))
 (segment (start 92.8 75.1) (end 94.7 73.2) (width 0.25) (layer "F.Cu") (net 3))
 (segment (start 84.87 63.73) (end 86.544 63.73) (width 0.25) (layer "F.Cu") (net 4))
 (segment (start 84.3 88) (end 88.5 92.2) (width 0.25) (layer "F.Cu") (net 4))
 (segment (start 84.3 64.3) (end 84.87 63.73) (width 0.25) (layer "F.Cu") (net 4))
 (segment (start 88.5 92.2) (end 95.55 92.2) (width 0.25) (layer "F.Cu") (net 4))
 (segment (start 84.3 68.3) (end 84.3 88) (width 0.25) (layer "F.Cu") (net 4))
 (via (at 84.3 68.3) (size 0.8) (drill 0.4) (layers "F.Cu" "B.Cu") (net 4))
 (via (at 84.3 64.3) (size 0.8) (drill 0.4) (layers "F.Cu" "B.Cu") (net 4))
 (segment (start 84.3 68.3) (end 84.3 64.3) (width 0.25) (layer "B.Cu") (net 4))
 (segment (start 91.584 66.27) (end 89.62452 68.22948) (width 0.25) (layer "F.Cu") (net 5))
 (segment (start 89.62452 68.22948) (end 89.62452 87.82452) (width 0.25) (layer "F.Cu") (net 5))
 (segment (start 89.62452 87.82452) (end 91.8 90) (width 0.25) (layer "F.Cu") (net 5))
 (segment (start 91.8 90) (end 95.55 90) (width 0.25) (layer "F.Cu") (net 5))
 (segment (start 82.604283 74.386805) (end 82.604283 88.504283) (width 0.25) (layer "F.Cu") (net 6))
 (segment (start 82.6 74.382522) (end 82.604283 74.386805) (width 0.25) (layer "F.Cu") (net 6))
 (segment (start 82.604283 69.033842) (end 82.6 69.038125) (width 0.25) (layer "F.Cu") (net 6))
 (segment (start 88.5 94.4) (end 95.55 94.4) (width 0.25) (layer "F.Cu") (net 6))
 (segment (start 82.6 68.2) (end 82.6 68.429353) (width 0.25) (layer "F.Cu") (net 6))
 (segment (start 84.53 66.27) (end 82.6 68.2) (width 0.25) (layer "F.Cu") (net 6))
 (segment (start 86.544 66.27) (end 84.53 66.27) (width 0.25) (layer "F.Cu") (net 6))
 (segment (start 82.6 69.038125) (end 82.6 74.382522) (width 0.25) (layer "F.Cu") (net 6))
 (segment (start 82.604283 68.433636) (end 82.604283 69.033842) (width 0.25) (layer "F.Cu") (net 6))
 (segment (start 82.6 68.429353) (end 82.604283 68.433636) (width 0.25) (layer "F.Cu") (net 6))
 (segment (start 82.604283 88.504283) (end 88.5 94.4) (width 0.25) (layer "F.Cu") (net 6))
 (segment (start 93.3 88.9) (end 95.55 88.9) (width 0.25) (layer "F.Cu") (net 7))
 (segment (start 91.584 87.184) (end 93.3 88.9) (width 0.25) (layer "F.Cu") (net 7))
 (segment (start 91.584 68.81) (end 91.584 87.184) (width 0.25) (layer "F.Cu") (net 7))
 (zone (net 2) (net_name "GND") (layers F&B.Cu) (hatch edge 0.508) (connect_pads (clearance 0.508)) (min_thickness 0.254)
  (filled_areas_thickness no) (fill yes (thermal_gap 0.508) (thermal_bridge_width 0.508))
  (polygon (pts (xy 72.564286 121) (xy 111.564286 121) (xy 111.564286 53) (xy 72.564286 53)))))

